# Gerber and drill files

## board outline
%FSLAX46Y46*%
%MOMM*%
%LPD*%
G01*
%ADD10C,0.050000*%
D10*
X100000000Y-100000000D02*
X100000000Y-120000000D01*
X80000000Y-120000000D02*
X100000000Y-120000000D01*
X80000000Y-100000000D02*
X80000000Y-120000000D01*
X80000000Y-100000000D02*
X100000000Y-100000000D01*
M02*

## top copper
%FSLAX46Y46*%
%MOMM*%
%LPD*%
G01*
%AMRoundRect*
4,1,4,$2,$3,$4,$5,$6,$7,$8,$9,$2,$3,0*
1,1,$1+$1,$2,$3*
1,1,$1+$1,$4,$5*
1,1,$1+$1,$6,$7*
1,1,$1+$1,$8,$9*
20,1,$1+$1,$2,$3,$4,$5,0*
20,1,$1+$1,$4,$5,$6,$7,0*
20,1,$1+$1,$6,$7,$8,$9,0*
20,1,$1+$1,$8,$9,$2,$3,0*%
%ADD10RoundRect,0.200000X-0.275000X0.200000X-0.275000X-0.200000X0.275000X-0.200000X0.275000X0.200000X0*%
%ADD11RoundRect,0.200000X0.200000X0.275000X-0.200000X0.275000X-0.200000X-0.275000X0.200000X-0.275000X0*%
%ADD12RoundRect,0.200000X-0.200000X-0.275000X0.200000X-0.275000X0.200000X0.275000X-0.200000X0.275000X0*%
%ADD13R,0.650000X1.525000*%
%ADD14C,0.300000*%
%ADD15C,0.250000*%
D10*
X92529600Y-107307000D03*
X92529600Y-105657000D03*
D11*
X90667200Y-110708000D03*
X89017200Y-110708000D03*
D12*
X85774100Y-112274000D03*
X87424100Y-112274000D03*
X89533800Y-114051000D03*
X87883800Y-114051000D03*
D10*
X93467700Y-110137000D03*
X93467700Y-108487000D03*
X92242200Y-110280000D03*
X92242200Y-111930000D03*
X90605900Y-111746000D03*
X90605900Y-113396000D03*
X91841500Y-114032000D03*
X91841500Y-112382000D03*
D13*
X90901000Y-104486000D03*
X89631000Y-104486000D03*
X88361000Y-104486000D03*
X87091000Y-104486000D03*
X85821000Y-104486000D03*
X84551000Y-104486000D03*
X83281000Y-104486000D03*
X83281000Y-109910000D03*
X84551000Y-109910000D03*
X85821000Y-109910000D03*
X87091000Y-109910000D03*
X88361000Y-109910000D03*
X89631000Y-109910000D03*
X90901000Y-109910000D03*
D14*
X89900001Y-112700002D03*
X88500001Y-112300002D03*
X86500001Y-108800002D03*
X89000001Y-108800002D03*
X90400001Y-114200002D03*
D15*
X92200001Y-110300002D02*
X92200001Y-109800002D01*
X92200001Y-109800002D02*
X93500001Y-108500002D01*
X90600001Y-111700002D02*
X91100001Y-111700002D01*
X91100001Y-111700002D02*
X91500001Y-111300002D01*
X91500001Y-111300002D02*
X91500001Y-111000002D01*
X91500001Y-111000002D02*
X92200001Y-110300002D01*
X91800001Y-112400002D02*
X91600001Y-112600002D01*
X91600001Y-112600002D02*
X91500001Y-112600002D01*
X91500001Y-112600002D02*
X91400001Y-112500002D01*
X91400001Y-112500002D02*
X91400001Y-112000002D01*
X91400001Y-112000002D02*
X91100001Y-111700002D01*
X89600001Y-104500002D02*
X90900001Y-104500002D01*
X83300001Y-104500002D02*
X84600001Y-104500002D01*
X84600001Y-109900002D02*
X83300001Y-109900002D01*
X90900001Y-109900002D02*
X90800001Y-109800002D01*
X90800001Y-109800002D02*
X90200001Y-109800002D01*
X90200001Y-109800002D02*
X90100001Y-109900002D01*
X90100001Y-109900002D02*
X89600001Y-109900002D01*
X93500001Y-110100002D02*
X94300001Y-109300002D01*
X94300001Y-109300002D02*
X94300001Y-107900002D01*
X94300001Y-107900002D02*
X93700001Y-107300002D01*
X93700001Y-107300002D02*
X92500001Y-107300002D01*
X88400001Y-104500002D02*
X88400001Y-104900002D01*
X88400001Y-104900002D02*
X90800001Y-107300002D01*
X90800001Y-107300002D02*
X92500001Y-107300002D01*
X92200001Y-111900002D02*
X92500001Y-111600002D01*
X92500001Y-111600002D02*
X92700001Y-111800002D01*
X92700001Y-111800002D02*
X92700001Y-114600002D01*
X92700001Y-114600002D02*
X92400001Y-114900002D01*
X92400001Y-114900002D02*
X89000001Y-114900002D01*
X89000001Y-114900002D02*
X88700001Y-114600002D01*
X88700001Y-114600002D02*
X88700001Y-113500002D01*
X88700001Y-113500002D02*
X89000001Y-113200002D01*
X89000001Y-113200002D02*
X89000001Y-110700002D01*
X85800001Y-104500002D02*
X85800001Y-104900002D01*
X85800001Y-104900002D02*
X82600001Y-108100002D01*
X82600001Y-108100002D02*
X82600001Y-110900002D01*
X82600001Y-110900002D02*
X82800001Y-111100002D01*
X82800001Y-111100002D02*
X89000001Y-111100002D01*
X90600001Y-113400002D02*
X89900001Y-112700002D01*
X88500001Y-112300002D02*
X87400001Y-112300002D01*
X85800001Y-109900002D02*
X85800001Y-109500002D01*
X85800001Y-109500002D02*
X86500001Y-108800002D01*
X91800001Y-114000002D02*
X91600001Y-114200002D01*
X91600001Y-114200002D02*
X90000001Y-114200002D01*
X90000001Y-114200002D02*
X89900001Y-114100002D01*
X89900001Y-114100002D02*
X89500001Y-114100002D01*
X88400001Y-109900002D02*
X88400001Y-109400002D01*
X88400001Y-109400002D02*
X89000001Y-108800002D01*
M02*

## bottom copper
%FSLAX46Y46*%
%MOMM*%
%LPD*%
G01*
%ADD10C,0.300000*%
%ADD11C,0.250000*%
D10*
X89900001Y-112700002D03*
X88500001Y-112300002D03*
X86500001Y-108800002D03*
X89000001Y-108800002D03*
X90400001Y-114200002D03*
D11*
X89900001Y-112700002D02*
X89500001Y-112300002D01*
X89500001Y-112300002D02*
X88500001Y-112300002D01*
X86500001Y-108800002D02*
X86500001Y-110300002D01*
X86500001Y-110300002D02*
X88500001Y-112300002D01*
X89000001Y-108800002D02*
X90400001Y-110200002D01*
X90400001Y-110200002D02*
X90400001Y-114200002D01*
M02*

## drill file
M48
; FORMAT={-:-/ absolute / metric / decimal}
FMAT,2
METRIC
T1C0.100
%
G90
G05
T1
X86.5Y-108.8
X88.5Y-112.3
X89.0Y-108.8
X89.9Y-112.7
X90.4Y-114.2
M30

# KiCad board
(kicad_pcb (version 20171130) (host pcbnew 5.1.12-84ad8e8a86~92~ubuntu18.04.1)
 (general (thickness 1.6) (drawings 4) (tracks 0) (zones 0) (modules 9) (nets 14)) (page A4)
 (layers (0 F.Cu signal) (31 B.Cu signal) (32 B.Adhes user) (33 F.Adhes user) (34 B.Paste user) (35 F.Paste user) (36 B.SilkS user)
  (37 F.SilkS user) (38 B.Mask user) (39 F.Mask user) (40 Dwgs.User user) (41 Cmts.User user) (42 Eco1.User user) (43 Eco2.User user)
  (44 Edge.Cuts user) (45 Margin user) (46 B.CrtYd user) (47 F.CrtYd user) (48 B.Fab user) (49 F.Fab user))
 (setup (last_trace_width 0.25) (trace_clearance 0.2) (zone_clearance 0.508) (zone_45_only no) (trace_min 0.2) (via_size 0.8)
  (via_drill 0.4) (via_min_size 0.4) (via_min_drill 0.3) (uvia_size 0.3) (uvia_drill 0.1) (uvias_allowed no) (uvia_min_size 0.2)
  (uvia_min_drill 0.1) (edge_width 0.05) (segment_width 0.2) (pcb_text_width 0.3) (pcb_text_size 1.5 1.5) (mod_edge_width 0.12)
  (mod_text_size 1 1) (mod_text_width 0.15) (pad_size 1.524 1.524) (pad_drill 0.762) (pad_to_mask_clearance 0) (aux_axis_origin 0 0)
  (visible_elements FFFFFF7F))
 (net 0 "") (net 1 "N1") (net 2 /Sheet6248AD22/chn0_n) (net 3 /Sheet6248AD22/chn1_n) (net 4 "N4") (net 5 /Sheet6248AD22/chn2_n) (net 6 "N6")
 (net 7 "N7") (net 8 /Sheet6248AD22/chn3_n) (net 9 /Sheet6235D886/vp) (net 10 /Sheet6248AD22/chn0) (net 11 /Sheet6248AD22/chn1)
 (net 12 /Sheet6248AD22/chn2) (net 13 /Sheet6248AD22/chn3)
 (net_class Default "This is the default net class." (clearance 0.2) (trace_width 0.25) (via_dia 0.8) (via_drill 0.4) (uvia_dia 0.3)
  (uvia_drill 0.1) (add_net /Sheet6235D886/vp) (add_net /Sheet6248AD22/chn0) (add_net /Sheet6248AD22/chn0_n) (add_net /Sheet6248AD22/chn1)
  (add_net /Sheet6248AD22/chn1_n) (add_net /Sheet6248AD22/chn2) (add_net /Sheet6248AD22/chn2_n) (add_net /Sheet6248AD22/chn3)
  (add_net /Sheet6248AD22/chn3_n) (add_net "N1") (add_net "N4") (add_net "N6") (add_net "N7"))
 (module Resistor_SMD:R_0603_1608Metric (layer F.Cu) (at 92.529600 106.482000 270.000000)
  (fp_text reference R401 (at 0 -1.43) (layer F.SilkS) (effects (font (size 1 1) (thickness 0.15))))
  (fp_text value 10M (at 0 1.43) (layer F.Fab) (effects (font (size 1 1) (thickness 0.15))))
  (pad 2 smd roundrect (at 0.825 0 270.000000) (size 0.8 0.95) (layers F.Cu F.Mask F.Paste) (roundrect_rratio 0.25) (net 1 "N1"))
  (pad 1 smd roundrect (at -0.825 0 270.000000) (size 0.8 0.95) (layers F.Cu F.Mask F.Paste) (roundrect_rratio 0.25)
   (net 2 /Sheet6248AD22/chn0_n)))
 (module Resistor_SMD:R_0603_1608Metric (layer F.Cu) (at 89.842200 110.708000 180.000000)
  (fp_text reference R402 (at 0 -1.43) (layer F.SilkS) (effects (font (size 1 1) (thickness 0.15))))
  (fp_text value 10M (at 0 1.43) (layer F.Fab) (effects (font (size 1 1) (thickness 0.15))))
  (pad 1 smd roundrect (at -0.825 0 180.000000) (size 0.8 0.95) (layers F.Cu F.Mask F.Paste) (roundrect_rratio 0.25)
   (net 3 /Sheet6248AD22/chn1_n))
  (pad 2 smd roundrect (at 0.825 0 180.000000) (size 0.8 0.95) (layers F.Cu F.Mask F.Paste) (roundrect_rratio 0.25) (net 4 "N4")))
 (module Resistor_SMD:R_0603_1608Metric (layer F.Cu) (at 86.599100 112.274000)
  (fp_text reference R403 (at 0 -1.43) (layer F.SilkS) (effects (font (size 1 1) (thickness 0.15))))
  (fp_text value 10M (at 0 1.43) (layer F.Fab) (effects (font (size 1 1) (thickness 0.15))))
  (pad 1 smd roundrect (at -0.825 0) (size 0.8 0.95) (layers F.Cu F.Mask F.Paste) (roundrect_rratio 0.25) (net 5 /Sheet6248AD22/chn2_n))
  (pad 2 smd roundrect (at 0.825 0) (size 0.8 0.95) (layers F.Cu F.Mask F.Paste) (roundrect_rratio 0.25) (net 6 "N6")))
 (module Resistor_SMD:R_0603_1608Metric (layer F.Cu) (at 88.708800 114.051000)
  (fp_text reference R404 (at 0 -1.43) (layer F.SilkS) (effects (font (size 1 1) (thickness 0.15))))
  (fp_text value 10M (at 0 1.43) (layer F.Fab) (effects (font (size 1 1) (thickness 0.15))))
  (pad 2 smd roundrect (at 0.825 0) (size 0.8 0.95) (layers F.Cu F.Mask F.Paste) (roundrect_rratio 0.25) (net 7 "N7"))
  (pad 1 smd roundrect (at -0.825 0) (size 0.8 0.95) (layers F.Cu F.Mask F.Paste) (roundrect_rratio 0.25) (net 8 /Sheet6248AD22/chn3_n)))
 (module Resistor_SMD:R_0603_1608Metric (layer F.Cu) (at 93.467700 109.312000 270.000000)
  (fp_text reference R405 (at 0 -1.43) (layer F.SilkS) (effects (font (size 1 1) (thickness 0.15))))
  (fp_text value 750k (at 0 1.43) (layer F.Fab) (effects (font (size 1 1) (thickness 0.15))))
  (pad 2 smd roundrect (at 0.825 0 270.000000) (size 0.8 0.95) (layers F.Cu F.Mask F.Paste) (roundrect_rratio 0.25) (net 1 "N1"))
  (pad 1 smd roundrect (at -0.825 0 270.000000) (size 0.8 0.95) (layers F.Cu F.Mask F.Paste) (roundrect_rratio 0.25)
   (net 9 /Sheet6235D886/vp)))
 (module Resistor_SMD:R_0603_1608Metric (layer F.Cu) (at 92.242200 111.105000 270.000000)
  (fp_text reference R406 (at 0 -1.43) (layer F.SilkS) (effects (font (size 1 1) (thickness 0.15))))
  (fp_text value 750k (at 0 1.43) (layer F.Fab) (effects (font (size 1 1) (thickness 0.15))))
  (pad 1 smd roundrect (at -0.825 0 270.000000) (size 0.8 0.95) (layers F.Cu F.Mask F.Paste) (roundrect_rratio 0.25)
   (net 9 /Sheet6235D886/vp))
  (pad 2 smd roundrect (at 0.825 0 270.000000) (size 0.8 0.95) (layers F.Cu F.Mask F.Paste) (roundrect_rratio 0.25) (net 4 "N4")))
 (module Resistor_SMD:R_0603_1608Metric (layer F.Cu) (at 90.605900 112.571000 270.000000)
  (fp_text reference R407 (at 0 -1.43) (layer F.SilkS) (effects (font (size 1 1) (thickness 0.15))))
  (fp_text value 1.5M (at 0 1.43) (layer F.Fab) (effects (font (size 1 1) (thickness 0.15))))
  (pad 1 smd roundrect (at -0.825 0 270.000000) (size 0.8 0.95) (layers F.Cu F.Mask F.Paste) (roundrect_rratio 0.25)
   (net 9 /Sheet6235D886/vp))
  (pad 2 smd roundrect (at 0.825 0 270.000000) (size 0.8 0.95) (layers F.Cu F.Mask F.Paste) (roundrect_rratio 0.25) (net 6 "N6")))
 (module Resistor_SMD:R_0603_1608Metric (layer F.Cu) (at 91.841500 113.207000 270.000000)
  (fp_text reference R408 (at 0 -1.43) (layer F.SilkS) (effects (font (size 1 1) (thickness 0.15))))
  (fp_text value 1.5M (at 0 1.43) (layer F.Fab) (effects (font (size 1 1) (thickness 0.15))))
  (pad 2 smd roundrect (at 0.825 0 270.000000) (size 0.8 0.95) (layers F.Cu F.Mask F.Paste) (roundrect_rratio 0.25) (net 7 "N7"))
  (pad 1 smd roundrect (at -0.825 0 270.000000) (size 0.8 0.95) (layers F.Cu F.Mask F.Paste) (roundrect_rratio 0.25)
   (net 9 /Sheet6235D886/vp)))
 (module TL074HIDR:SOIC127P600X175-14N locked (layer F.Cu) (at 87.091000 107.198000 270.000000)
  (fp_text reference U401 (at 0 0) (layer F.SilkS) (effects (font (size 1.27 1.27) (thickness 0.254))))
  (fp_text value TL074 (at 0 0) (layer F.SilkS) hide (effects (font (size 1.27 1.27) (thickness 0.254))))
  (pad 1 smd rect (at -2.712 -3.81) (size 0.65 1.525) (layers F.Cu F.Mask F.Paste) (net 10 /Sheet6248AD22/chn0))
  (pad 2 smd rect (at -2.712 -2.54) (size 0.65 1.525) (layers F.Cu F.Mask F.Paste) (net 10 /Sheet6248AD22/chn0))
  (pad 3 smd rect (at -2.712 -1.27) (size 0.65 1.525) (layers F.Cu F.Mask F.Paste) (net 1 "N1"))
  (pad 4 smd rect (at -2.712 0) (size 0.65 1.525) (layers F.Cu F.Mask F.Paste))
  (pad 5 smd rect (at -2.712 1.27) (size 0.65 1.525) (layers F.Cu F.Mask F.Paste) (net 4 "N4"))
  (pad 6 smd rect (at -2.712 2.54) (size 0.65 1.525) (layers F.Cu F.Mask F.Paste) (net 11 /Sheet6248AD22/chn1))
  (pad 7 smd rect (at -2.712 3.81) (size 0.65 1.525) (layers F.Cu F.Mask F.Paste) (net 11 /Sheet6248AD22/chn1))
  (pad 8 smd rect (at 2.712 3.81) (size 0.65 1.525) (layers F.Cu F.Mask F.Paste) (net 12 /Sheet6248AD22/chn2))
  (pad 9 smd rect (at 2.712 2.54) (size 0.65 1.525) (layers F.Cu F.Mask F.Paste) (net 12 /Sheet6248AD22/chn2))
  (pad 10 smd rect (at 2.712 1.27) (size 0.65 1.525) (layers F.Cu F.Mask F.Paste) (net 6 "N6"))
  (pad 11 smd rect (at 2.712 0) (size 0.65 1.525) (layers F.Cu F.Mask F.Paste))
  (pad 12 smd rect (at 2.712 -1.27) (size 0.65 1.525) (layers F.Cu F.Mask F.Paste) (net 7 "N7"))
  (pad 13 smd rect (at 2.712 -2.54) (size 0.65 1.525) (layers F.Cu F.Mask F.Paste) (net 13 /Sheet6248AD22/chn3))
  (pad 14 smd rect (at 2.712 -3.81) (size 0.65 1.525) (layers F.Cu F.Mask F.Paste) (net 13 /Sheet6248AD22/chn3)))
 (gr_line (start 100 100) (end 100 120) (layer Edge.Cuts) (width 0.05))
 (gr_line (start 80 120) (end 100 120) (layer Edge.Cuts) (width 0.05))
 (gr_line (start 80 100) (end 80 120) (layer Edge.Cuts) (width 0.05))
 (gr_line (start 80 100) (end 100 100) (layer Edge.Cuts) (width 0.05))
 (segment (start 92.200001 110.300002) (end 92.200001 109.800002) (width 0.250000) (layer F.Cu) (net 9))
 (segment (start 92.200001 109.800002) (end 93.500001 108.500002) (width 0.250000) (layer F.Cu) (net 9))
 (segment (start 90.600001 111.700002) (end 91.100001 111.700002) (width 0.250000) (layer F.Cu) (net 9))
 (segment (start 91.100001 111.700002) (end 91.500001 111.300002) (width 0.250000) (layer F.Cu) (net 9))
 (segment (start 91.500001 111.300002) (end 91.500001 111.000002) (width 0.250000) (layer F.Cu) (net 9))
 (segment (start 91.500001 111.000002) (end 92.200001 110.300002) (width 0.250000) (layer F.Cu) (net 9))
 (segment (start 91.800001 112.400002) (end 91.600001 112.600002) (width 0.250000) (layer F.Cu) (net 9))
 (segment (start 91.600001 112.600002) (end 91.500001 112.600002) (width 0.250000) (layer F.Cu) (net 9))
 (segment (start 91.500001 112.600002) (end 91.400001 112.500002) (width 0.250000) (layer F.Cu) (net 9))
 (segment (start 91.400001 112.500002) (end 91.400001 112.000002) (width 0.250000) (layer F.Cu) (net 9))
 (segment (start 91.400001 112.000002) (end 91.100001 111.700002) (width 0.250000) (layer F.Cu) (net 9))
 (segment (start 89.600001 104.500002) (end 90.900001 104.500002) (width 0.250000) (layer F.Cu) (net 10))
 (segment (start 83.300001 104.500002) (end 84.600001 104.500002) (width 0.250000) (layer F.Cu) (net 11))
 (segment (start 84.600001 109.900002) (end 83.300001 109.900002) (width 0.250000) (layer F.Cu) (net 12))
 (segment (start 90.900001 109.900002) (end 90.800001 109.800002) (width 0.250000) (layer F.Cu) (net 13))
 (segment (start 90.800001 109.800002) (end 90.200001 109.800002) (width 0.250000) (layer F.Cu) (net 13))
 (segment (start 90.200001 109.800002) (end 90.100001 109.900002) (width 0.250000) (layer F.Cu) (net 13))
 (segment (start 90.100001 109.900002) (end 89.600001 109.900002) (width 0.250000) (layer F.Cu) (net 13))
 (segment (start 93.500001 110.100002) (end 94.300001 109.300002) (width 0.250000) (layer F.Cu) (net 1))
 (segment (start 94.300001 109.300002) (end 94.300001 107.900002) (width 0.250000) (layer F.Cu) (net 1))
 (segment (start 94.300001 107.900002) (end 93.700001 107.300002) (width 0.250000) (layer F.Cu) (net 1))
 (segment (start 93.700001 107.300002) (end 92.500001 107.300002) (width 0.250000) (layer F.Cu) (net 1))
 (segment (start 88.400001 104.500002) (end 88.400001 104.900002) (width 0.250000) (layer F.Cu) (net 1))
 (segment (start 88.400001 104.900002) (end 90.800001 107.300002) (width 0.250000) (layer F.Cu) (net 1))
 (segment (start 90.800001 107.300002) (end 92.500001 107.300002) (width 0.250000) (layer F.Cu) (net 1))
 (segment (start 92.200001 111.900002) (end 92.500001 111.600002) (width 0.250000) (layer F.Cu) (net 4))
 (segment (start 92.500001 111.600002) (end 92.700001 111.800002) (width 0.250000) (layer F.Cu) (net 4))
 (segment (start 92.700001 111.800002) (end 92.700001 114.600002) (width 0.250000) (layer F.Cu) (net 4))
 (segment (start 92.700001 114.600002) (end 92.400001 114.900002) (width 0.250000) (layer F.Cu) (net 4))
 (segment (start 92.400001 114.900002) (end 89.000001 114.900002) (width 0.250000) (layer F.Cu) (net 4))
 (segment (start 89.000001 114.900002) (end 88.700001 114.600002) (width 0.250000) (layer F.Cu) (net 4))
 (segment (start 88.700001 114.600002) (end 88.700001 113.500002) (width 0.250000) (layer F.Cu) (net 4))
 (segment (start 88.700001 113.500002) (end 89.000001 113.200002) (width 0.250000) (layer F.Cu) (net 4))
 (segment (start 89.000001 113.200002) (end 89.000001 110.700002) (width 0.250000) (layer F.Cu) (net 4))
 (segment (start 85.800001 104.500002) (end 85.800001 104.900002) (width 0.250000) (layer F.Cu) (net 4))
 (segment (start 85.800001 104.900002) (end 82.600001 108.100002) (width 0.250000) (layer F.Cu) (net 4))
 (segment (start 82.600001 108.100002) (end 82.600001 110.900002) (width 0.250000) (layer F.Cu) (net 4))
 (segment (start 82.600001 110.900002) (end 82.800001 111.100002) (width 0.250000) (layer F.Cu) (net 4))
 (segment (start 82.800001 111.100002) (end 89.000001 111.100002) (width 0.250000) (layer F.Cu) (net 4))
 (segment (start 90.600001 113.400002) (end 89.900001 112.700002) (width 0.250000) (layer F.Cu) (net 6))
 (segment (start 89.900001 112.700002) (end 89.500001 112.300002) (width 0.250000) (layer B.Cu) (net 6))
 (segment (start 89.500001 112.300002) (end 88.500001 112.300002) (width 0.250000) (layer B.Cu) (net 6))
 (segment (start 88.500001 112.300002) (end 87.400001 112.300002) (width 0.250000) (layer F.Cu) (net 6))
 (segment (start 85.800001 109.900002) (end 85.800001 109.500002) (width 0.250000) (layer F.Cu) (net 6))
 (segment (start 85.800001 109.500002) (end 86.500001 108.800002) (width 0.250000) (layer F.Cu) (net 6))
 (segment (start 86.500001 108.800002) (end 86.500001 110.300002) (width 0.250000) (layer B.Cu) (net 6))
 (segment (start 86.500001 110.300002) (end 88.500001 112.300002) (width 0.250000) (layer B.Cu) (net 6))
 (via micro (at 89.900001 112.700002) (size 0.300000) (drill 0.100000) (layers F.Cu B.Cu) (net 6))
 (via micro (at 88.500001 112.300002) (size 0.300000) (drill 0.100000) (layers F.Cu B.Cu) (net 6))
 (via micro (at 86.500001 108.800002) (size 0.300000) (drill 0.100000) (layers F.Cu B.Cu) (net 6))
 (segment (start 91.800001 114.000002) (end 91.600001 114.200002) (width 0.250000) (layer F.Cu) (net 7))
 (segment (start 91.600001 114.200002) (end 90.000001 114.200002) (width 0.250000) (layer F.Cu) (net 7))
 (segment (start 90.000001 114.200002) (end 89.900001 114.100002) (width 0.250000) (layer F.Cu) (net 7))
 (segment (start 89.900001 114.100002) (end 89.500001 114.100002) (width 0.250000) (layer F.Cu) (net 7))
 (segment (start 88.400001 109.900002) (end 88.400001 109.400002) (width 0.250000) (layer F.Cu) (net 7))
 (segment (start 88.400001 109.400002) (end 89.000001 108.800002) (width 0.250000) (layer F.Cu) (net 7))
 (segment (start 89.000001 108.800002) (end 90.400001 110.200002) (width 0.250000) (layer B.Cu) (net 7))
 (segment (start 90.400001 110.200002) (end 90.400001 114.200002) (width 0.250000) (layer B.Cu) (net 7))
 (via micro (at 89.000001 108.800002) (size 0.300000) (drill 0.100000) (layers F.Cu B.Cu) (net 7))
 (via micro (at 90.400001 114.200002) (size 0.300000) (drill 0.100000) (layers F.Cu B.Cu) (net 7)))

